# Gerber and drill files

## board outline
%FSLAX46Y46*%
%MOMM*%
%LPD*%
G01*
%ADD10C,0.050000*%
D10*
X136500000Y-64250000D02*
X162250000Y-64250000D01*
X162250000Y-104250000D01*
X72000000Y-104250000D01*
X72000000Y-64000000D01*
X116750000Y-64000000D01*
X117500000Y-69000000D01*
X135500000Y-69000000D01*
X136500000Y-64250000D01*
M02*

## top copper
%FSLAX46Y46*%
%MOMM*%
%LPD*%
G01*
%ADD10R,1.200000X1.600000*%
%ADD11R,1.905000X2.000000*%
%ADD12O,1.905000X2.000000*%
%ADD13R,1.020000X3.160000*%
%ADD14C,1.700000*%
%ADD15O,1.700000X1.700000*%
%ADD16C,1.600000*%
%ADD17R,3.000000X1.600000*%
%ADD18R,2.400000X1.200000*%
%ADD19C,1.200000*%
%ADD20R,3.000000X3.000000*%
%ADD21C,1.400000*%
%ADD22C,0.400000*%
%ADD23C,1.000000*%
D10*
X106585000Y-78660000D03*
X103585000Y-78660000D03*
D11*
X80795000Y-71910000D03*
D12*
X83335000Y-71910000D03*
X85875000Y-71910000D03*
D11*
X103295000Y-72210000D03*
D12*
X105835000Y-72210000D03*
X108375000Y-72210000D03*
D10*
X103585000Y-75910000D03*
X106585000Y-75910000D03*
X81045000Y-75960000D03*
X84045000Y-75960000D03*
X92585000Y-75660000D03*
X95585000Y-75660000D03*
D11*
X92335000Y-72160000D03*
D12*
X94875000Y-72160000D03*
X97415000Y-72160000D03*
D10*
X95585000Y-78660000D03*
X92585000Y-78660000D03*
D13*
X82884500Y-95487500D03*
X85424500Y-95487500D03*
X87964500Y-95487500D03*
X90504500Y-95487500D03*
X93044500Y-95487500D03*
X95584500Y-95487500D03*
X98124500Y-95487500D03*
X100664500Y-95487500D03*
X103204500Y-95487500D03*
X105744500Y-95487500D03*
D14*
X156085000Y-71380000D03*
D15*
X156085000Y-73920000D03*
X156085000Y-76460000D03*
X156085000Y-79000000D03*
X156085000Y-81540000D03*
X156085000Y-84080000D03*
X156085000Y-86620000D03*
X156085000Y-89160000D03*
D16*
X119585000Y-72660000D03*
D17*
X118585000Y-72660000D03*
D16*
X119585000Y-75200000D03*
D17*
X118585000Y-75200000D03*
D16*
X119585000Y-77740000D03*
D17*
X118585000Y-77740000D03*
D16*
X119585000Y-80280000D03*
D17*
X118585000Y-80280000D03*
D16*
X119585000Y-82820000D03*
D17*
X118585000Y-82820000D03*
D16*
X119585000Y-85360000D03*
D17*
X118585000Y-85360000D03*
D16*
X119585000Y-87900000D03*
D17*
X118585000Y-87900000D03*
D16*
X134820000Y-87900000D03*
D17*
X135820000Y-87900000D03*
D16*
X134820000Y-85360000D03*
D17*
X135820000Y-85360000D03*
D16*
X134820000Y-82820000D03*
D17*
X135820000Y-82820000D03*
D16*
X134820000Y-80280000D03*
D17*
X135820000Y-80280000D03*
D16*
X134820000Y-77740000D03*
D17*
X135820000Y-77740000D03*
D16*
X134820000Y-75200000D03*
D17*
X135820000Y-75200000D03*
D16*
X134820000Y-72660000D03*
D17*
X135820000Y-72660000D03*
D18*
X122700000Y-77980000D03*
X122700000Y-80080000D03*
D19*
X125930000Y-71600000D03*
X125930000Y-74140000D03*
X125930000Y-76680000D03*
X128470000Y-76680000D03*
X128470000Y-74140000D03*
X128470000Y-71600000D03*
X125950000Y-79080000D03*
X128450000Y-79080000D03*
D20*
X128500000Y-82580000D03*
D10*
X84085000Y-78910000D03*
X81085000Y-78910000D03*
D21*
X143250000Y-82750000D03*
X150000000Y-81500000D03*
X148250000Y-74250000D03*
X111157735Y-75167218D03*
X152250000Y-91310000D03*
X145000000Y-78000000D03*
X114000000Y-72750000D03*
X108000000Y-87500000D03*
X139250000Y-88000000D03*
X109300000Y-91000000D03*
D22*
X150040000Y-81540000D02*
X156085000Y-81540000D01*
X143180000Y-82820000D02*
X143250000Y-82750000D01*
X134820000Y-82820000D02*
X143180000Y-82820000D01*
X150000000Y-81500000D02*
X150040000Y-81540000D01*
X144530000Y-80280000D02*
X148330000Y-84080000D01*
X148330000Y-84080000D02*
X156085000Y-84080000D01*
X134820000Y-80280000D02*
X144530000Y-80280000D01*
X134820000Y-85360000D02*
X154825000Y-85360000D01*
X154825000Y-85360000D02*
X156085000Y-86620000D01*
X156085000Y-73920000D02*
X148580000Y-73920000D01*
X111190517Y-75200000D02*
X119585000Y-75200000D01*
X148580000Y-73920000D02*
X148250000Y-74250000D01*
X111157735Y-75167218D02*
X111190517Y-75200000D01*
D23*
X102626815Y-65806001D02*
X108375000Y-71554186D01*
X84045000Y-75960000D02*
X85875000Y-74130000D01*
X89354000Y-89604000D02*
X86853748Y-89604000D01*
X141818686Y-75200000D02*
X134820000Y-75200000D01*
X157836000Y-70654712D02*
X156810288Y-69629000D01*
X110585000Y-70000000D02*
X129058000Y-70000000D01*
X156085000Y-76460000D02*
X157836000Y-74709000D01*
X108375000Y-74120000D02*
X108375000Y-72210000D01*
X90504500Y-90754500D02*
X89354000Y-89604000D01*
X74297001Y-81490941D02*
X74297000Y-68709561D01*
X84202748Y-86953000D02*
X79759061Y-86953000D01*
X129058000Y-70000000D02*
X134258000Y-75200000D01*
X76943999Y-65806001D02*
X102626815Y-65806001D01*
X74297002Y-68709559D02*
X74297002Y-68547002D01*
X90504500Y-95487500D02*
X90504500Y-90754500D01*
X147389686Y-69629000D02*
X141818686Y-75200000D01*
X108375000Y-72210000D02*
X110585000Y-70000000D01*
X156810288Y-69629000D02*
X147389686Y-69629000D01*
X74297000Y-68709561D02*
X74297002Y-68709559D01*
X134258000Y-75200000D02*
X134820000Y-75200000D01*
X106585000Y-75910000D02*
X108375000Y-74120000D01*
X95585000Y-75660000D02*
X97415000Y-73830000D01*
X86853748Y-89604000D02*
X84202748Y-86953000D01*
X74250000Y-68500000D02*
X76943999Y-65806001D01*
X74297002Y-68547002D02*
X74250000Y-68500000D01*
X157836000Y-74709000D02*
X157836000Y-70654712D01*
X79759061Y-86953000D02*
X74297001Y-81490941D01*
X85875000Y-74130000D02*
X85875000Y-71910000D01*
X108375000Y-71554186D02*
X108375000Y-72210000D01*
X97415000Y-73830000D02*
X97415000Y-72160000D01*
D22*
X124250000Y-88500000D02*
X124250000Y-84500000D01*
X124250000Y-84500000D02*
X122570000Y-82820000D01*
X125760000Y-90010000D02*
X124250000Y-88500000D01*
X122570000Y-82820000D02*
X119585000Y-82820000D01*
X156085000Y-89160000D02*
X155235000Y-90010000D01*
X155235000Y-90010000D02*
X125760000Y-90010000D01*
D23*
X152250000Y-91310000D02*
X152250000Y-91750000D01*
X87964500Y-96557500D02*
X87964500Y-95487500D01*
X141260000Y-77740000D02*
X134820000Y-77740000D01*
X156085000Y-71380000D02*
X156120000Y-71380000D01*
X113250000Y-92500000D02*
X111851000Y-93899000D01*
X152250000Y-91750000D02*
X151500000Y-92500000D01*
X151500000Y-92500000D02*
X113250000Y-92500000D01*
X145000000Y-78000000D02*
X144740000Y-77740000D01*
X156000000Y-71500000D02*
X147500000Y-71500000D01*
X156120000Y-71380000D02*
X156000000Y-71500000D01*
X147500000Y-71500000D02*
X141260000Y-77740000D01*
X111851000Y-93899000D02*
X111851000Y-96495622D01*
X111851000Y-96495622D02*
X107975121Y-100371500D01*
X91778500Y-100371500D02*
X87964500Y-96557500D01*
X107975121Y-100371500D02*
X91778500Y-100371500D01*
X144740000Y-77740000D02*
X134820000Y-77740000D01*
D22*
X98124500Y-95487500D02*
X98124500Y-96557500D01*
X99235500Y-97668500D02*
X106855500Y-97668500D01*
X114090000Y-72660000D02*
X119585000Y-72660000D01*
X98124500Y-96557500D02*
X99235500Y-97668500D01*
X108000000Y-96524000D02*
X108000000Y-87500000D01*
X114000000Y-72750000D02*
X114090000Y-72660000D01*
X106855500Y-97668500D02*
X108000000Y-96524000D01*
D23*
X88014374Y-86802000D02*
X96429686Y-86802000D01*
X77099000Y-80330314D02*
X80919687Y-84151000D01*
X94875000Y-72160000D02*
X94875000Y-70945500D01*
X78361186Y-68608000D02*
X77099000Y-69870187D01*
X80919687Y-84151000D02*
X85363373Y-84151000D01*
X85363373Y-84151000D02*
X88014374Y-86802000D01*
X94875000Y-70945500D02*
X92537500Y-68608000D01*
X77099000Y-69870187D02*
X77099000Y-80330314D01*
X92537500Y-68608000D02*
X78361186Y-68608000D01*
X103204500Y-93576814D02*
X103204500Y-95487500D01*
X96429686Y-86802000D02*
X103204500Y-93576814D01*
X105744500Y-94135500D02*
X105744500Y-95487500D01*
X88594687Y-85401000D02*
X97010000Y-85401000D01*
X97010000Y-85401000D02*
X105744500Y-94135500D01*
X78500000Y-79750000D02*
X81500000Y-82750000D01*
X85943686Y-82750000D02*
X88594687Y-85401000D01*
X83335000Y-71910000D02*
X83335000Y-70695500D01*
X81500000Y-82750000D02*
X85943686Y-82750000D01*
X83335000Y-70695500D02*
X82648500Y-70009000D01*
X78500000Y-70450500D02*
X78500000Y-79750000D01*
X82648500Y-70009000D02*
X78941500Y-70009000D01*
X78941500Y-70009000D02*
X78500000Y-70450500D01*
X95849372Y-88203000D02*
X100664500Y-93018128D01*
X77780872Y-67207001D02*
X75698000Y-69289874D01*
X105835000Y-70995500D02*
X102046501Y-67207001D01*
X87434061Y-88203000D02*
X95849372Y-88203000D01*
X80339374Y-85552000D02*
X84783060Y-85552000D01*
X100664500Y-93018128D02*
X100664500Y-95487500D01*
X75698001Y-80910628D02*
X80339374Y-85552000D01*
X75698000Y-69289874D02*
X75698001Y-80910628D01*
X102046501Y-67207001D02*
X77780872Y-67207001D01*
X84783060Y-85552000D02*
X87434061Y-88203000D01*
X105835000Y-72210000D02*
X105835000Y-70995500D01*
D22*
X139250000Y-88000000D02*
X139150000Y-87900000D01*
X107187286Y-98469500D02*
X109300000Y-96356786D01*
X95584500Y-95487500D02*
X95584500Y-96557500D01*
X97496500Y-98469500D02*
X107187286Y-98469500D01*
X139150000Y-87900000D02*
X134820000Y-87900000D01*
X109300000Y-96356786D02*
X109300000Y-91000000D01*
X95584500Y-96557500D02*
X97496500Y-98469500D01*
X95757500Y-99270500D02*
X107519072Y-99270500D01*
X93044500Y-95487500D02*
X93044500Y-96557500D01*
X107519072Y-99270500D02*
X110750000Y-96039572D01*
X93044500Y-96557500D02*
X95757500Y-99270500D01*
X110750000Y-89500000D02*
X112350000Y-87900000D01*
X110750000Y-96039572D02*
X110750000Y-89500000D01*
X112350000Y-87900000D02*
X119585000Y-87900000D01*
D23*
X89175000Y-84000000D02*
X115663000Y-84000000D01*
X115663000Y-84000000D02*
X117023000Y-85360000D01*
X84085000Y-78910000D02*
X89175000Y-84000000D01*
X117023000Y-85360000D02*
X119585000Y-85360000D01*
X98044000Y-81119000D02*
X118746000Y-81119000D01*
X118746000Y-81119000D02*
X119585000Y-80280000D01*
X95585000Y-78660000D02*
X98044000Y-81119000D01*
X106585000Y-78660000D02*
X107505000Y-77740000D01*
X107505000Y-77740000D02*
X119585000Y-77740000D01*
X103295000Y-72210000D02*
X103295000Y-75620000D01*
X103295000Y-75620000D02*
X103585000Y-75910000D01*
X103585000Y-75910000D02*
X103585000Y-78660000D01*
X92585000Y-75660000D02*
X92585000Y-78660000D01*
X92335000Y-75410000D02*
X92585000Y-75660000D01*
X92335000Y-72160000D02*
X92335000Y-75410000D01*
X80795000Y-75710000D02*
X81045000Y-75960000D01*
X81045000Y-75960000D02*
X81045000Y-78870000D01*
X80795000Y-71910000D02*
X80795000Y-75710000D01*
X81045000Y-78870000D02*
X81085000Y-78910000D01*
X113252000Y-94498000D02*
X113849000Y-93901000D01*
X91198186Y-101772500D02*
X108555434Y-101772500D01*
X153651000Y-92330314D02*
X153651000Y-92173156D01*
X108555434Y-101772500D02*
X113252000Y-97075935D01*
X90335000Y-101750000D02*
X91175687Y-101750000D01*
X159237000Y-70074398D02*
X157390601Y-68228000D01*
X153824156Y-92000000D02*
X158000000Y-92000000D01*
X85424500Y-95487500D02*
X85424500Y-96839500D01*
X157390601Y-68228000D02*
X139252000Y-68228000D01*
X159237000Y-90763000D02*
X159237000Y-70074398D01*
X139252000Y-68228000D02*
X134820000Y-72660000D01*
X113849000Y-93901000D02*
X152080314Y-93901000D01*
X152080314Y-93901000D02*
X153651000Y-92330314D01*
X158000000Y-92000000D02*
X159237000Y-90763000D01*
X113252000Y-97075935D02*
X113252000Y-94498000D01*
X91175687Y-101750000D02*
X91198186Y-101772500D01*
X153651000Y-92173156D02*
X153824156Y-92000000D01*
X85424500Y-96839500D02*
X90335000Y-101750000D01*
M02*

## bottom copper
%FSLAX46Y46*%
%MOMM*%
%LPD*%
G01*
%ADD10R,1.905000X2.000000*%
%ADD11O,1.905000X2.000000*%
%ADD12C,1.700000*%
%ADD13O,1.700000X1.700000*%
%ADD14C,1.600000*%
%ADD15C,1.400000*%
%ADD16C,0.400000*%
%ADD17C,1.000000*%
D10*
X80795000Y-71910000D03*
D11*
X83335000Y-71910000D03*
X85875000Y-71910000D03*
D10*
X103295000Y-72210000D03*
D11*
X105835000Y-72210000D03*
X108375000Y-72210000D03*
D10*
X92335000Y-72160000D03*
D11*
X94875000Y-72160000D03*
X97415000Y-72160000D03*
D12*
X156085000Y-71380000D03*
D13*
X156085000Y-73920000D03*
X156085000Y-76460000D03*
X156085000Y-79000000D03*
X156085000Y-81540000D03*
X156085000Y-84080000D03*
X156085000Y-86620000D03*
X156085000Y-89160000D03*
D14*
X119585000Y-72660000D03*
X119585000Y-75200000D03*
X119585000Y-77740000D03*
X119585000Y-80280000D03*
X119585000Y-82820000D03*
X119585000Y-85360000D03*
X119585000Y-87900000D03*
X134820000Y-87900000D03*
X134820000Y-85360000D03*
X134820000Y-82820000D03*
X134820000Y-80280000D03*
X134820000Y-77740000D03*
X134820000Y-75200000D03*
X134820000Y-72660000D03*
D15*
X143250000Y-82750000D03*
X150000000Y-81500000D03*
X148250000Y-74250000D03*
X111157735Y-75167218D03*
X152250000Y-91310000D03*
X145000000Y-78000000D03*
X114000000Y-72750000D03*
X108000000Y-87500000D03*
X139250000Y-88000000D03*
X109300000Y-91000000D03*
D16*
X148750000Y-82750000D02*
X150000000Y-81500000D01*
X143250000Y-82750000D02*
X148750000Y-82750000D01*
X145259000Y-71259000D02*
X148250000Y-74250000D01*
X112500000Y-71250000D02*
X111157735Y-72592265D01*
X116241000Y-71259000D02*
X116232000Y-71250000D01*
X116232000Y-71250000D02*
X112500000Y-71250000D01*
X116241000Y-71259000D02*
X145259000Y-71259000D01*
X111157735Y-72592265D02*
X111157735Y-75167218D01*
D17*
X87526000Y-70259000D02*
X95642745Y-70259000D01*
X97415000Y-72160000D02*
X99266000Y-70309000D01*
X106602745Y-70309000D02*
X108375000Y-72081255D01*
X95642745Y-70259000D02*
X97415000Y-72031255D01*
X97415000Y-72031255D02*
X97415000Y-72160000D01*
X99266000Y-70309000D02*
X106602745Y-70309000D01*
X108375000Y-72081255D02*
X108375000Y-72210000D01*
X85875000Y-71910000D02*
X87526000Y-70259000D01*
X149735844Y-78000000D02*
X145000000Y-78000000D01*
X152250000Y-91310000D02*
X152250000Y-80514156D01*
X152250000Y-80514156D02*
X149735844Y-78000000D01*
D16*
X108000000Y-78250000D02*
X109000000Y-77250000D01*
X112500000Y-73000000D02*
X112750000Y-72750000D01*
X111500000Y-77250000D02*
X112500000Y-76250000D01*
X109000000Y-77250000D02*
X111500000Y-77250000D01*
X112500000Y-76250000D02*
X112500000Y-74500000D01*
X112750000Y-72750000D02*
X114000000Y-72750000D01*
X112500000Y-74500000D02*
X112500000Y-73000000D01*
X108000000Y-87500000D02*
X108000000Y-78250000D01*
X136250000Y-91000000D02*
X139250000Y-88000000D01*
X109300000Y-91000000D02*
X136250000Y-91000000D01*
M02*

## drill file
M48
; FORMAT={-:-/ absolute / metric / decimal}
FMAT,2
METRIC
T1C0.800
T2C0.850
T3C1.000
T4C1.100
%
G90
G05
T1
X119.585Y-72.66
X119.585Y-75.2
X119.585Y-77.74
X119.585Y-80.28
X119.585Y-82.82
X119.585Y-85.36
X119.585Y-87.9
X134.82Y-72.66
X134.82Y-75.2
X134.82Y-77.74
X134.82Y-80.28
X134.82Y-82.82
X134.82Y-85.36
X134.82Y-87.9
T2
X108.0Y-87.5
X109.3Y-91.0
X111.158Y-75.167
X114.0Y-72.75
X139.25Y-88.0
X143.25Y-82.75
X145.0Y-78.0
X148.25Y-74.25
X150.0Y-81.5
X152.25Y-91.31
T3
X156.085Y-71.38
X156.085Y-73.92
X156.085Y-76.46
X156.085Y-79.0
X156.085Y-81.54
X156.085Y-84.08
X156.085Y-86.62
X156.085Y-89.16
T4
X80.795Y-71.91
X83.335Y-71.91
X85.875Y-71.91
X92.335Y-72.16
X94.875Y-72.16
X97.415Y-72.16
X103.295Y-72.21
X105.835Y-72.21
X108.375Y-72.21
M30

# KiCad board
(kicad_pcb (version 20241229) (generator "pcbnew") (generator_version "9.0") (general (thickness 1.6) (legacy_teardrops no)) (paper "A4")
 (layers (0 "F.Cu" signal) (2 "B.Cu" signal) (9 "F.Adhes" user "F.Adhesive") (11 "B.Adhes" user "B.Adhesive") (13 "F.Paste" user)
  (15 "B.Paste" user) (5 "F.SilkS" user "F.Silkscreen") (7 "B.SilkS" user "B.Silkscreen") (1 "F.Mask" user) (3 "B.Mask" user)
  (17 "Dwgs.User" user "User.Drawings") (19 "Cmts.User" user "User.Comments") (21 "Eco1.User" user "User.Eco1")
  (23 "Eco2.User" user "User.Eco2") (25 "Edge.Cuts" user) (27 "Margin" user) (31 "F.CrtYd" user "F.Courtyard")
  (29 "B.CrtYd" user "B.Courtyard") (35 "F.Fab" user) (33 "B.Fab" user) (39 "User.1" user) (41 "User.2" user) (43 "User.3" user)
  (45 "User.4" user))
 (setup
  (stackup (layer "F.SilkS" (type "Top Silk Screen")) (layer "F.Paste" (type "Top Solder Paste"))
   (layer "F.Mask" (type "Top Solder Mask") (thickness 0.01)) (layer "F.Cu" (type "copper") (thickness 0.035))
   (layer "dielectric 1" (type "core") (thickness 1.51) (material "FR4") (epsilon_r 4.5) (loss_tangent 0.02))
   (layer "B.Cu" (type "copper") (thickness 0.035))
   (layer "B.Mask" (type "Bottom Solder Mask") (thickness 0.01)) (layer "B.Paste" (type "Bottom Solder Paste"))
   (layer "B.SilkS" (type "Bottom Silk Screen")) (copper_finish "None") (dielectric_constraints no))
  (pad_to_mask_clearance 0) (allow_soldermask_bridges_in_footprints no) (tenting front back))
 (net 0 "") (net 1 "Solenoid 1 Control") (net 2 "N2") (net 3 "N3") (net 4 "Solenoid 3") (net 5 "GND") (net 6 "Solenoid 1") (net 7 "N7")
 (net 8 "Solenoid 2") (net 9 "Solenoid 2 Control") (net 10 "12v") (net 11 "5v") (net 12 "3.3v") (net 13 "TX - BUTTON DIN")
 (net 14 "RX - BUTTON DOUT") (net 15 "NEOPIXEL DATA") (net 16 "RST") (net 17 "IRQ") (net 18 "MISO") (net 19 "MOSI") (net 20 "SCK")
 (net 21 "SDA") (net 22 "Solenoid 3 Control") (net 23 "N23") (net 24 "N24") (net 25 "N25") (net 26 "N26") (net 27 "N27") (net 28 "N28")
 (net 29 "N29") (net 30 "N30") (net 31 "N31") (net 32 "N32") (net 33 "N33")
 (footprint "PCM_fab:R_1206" (layer "F.Cu") (at 105.085 78.66 180)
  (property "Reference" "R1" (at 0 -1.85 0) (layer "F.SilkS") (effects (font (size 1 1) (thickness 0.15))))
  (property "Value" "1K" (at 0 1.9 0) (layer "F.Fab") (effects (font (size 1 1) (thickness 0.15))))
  (pad "1" smd rect (at -1.5 0 180) (size 1.2 1.6) (layers "F.Cu" "F.Mask" "F.Paste") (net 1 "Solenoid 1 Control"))
  (pad "2" smd rect (at 1.5 0 180) (size 1.2 1.6) (layers "F.Cu" "F.Mask" "F.Paste") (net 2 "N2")))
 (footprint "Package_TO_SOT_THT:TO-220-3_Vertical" (layer "F.Cu") (at 80.795 71.91)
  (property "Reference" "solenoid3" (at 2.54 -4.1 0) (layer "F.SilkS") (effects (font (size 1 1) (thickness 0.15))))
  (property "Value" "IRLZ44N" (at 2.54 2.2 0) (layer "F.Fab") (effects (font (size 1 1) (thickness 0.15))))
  (pad "1" thru_hole rect (at 0 0) (size 1.905 2) (drill 1.1) (layers "*.Cu" "*.Mask") (remove_unused_layers no) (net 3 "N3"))
  (pad "2" thru_hole oval (at 2.54 0) (size 1.905 2) (drill 1.1) (layers "*.Cu" "*.Mask") (remove_unused_layers no) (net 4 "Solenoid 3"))
  (pad "3" thru_hole oval (at 5.08 0) (size 1.905 2) (drill 1.1) (layers "*.Cu" "*.Mask") (remove_unused_layers no) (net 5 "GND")))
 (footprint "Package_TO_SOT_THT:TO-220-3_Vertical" (layer "F.Cu") (at 103.295 72.21)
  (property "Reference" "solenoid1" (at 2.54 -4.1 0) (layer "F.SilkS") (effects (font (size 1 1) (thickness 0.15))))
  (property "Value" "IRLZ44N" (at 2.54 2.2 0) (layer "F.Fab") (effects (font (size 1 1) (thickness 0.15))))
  (pad "1" thru_hole rect (at 0 0) (size 1.905 2) (drill 1.1) (layers "*.Cu" "*.Mask") (remove_unused_layers no) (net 2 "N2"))
  (pad "2" thru_hole oval (at 2.54 0) (size 1.905 2) (drill 1.1) (layers "*.Cu" "*.Mask") (remove_unused_layers no) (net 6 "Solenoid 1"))
  (pad "3" thru_hole oval (at 5.08 0) (size 1.905 2) (drill 1.1) (layers "*.Cu" "*.Mask") (remove_unused_layers no) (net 5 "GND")))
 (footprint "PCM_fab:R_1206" (layer "F.Cu") (at 105.085 75.91)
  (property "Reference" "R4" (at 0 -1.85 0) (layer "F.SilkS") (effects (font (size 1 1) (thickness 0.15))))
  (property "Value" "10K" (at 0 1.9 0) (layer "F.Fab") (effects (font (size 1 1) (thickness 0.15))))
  (pad "1" smd rect (at -1.5 0) (size 1.2 1.6) (layers "F.Cu" "F.Mask" "F.Paste") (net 2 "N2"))
  (pad "2" smd rect (at 1.5 0) (size 1.2 1.6) (layers "F.Cu" "F.Mask" "F.Paste") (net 5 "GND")))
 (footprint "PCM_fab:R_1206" (layer "F.Cu") (at 82.545 75.96)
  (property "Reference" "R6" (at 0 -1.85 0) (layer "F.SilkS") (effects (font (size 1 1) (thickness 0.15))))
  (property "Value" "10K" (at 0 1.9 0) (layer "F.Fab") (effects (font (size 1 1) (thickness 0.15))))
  (pad "1" smd rect (at -1.5 0) (size 1.2 1.6) (layers "F.Cu" "F.Mask" "F.Paste") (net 3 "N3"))
  (pad "2" smd rect (at 1.5 0) (size 1.2 1.6) (layers "F.Cu" "F.Mask" "F.Paste") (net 5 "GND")))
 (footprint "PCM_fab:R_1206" (layer "F.Cu") (at 94.085 75.66)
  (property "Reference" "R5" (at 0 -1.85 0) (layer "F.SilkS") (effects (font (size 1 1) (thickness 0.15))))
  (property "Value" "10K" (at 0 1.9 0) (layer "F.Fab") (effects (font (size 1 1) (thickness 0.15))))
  (pad "1" smd rect (at -1.5 0) (size 1.2 1.6) (layers "F.Cu" "F.Mask" "F.Paste") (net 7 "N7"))
  (pad "2" smd rect (at 1.5 0) (size 1.2 1.6) (layers "F.Cu" "F.Mask" "F.Paste") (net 5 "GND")))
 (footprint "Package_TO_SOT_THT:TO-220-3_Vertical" (layer "F.Cu") (at 92.335 72.16)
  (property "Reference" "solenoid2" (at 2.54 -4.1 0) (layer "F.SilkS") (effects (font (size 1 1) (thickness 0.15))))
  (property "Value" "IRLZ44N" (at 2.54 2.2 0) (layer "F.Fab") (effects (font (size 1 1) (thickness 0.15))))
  (pad "1" thru_hole rect (at 0 0) (size 1.905 2) (drill 1.1) (layers "*.Cu" "*.Mask") (remove_unused_layers no) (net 7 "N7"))
  (pad "2" thru_hole oval (at 2.54 0) (size 1.905 2) (drill 1.1) (layers "*.Cu" "*.Mask") (remove_unused_layers no) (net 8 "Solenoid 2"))
  (pad "3" thru_hole oval (at 5.08 0) (size 1.905 2) (drill 1.1) (layers "*.Cu" "*.Mask") (remove_unused_layers no) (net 5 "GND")))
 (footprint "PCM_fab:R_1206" (layer "F.Cu") (at 94.085 78.66 180)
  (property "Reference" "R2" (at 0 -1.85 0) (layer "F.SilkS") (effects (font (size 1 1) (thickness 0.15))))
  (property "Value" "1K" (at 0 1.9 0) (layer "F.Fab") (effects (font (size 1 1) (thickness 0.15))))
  (pad "1" smd rect (at -1.5 0 180) (size 1.2 1.6) (layers "F.Cu" "F.Mask" "F.Paste") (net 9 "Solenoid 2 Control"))
  (pad "2" smd rect (at 1.5 0 180) (size 1.2 1.6) (layers "F.Cu" "F.Mask" "F.Paste") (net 7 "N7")))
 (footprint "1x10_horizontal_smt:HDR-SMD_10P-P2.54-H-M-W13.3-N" (layer "F.Cu") (at 94.3145 95.4875)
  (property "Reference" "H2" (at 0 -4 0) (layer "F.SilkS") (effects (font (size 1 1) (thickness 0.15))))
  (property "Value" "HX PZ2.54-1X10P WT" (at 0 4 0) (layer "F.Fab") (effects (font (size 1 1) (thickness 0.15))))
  (pad "1" smd rect (at -11.43 0) (size 1.02 3.16) (layers "F.Cu" "F.Mask" "F.Paste") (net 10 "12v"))
  (pad "2" smd rect (at -8.89 0) (size 1.02 3.16) (layers "F.Cu" "F.Mask" "F.Paste") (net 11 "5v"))
  (pad "3" smd rect (at -6.35 0) (size 1.02 3.16) (layers "F.Cu" "F.Mask" "F.Paste") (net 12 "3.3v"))
  (pad "4" smd rect (at -3.81 0) (size 1.02 3.16) (layers "F.Cu" "F.Mask" "F.Paste") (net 5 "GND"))
  (pad "5" smd rect (at -1.27 0) (size 1.02 3.16) (layers "F.Cu" "F.Mask" "F.Paste") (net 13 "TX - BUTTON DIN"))
  (pad "6" smd rect (at 1.27 0) (size 1.02 3.16) (layers "F.Cu" "F.Mask" "F.Paste") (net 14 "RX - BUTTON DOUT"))
  (pad "7" smd rect (at 3.81 0) (size 1.02 3.16) (layers "F.Cu" "F.Mask" "F.Paste") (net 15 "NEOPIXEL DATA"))
  (pad "8" smd rect (at 6.35 0) (size 1.02 3.16) (layers "F.Cu" "F.Mask" "F.Paste") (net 6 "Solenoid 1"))
  (pad "9" smd rect (at 8.89 0) (size 1.02 3.16) (layers "F.Cu" "F.Mask" "F.Paste") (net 8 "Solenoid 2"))
  (pad "10" smd rect (at 11.43 0) (size 1.02 3.16) (layers "F.Cu" "F.Mask" "F.Paste") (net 4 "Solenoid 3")))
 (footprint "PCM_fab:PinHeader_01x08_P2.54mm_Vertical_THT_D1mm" (layer "F.Cu") (at 156.085 71.38)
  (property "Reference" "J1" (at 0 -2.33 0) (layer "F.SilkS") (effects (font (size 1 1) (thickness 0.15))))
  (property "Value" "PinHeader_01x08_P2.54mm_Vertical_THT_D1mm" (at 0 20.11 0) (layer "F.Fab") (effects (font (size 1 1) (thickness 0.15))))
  (pad "1" thru_hole circle (at 0 0) (size 1.7 1.7) (drill 1) (layers "*.Cu" "*.Mask") (remove_unused_layers no) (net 12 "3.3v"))
  (pad "2" thru_hole oval (at 0 2.54) (size 1.7 1.7) (drill 1) (layers "*.Cu" "*.Mask") (remove_unused_layers no) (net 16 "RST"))
  (pad "3" thru_hole oval (at 0 5.08) (size 1.7 1.7) (drill 1) (layers "*.Cu" "*.Mask") (remove_unused_layers no) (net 5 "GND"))
  (pad "4" thru_hole oval (at 0 7.62) (size 1.7 1.7) (drill 1) (layers "*.Cu" "*.Mask") (remove_unused_layers no) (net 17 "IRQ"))
  (pad "5" thru_hole oval (at 0 10.16) (size 1.7 1.7) (drill 1) (layers "*.Cu" "*.Mask") (remove_unused_layers no) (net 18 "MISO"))
  (pad "6" thru_hole oval (at 0 12.7) (size 1.7 1.7) (drill 1) (layers "*.Cu" "*.Mask") (remove_unused_layers no) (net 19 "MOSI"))
  (pad "7" thru_hole oval (at 0 15.24) (size 1.7 1.7) (drill 1) (layers "*.Cu" "*.Mask") (remove_unused_layers no) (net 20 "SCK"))
  (pad "8" thru_hole oval (at 0 17.78) (size 1.7 1.7) (drill 1) (layers "*.Cu" "*.Mask") (remove_unused_layers no) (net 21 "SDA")))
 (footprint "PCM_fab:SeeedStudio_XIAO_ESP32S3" (layer "F.Cu") (at 127.2 80.28)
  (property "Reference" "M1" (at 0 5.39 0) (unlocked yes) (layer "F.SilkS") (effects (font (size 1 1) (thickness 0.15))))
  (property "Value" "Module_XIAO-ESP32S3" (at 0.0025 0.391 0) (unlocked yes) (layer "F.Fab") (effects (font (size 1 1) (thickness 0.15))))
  (pad "1" thru_hole circle (at -7.615 -7.62) (size 1.6 1.6) (drill 0.8) (layers "*.Cu" "*.Mask") (remove_unused_layers no)
   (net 15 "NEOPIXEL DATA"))
  (pad "1" smd rect (at -7.615 -7.62) (size 3 1.6) (drill (offset -1 0)) (layers "F.Cu" "F.Mask" "F.Paste") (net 15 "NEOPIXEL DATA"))
  (pad "2" thru_hole circle (at -7.615 -5.08) (size 1.6 1.6) (drill 0.8) (layers "*.Cu" "*.Mask") (remove_unused_layers no) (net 16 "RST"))
  (pad "2" smd rect (at -7.615 -5.08) (size 3 1.6) (drill (offset -1 0)) (layers "F.Cu" "F.Mask" "F.Paste") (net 16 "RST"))
  (pad "3" thru_hole circle (at -7.615 -2.54) (size 1.6 1.6) (drill 0.8) (layers "*.Cu" "*.Mask") (remove_unused_layers no)
   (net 1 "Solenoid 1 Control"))
  (pad "3" smd rect (at -7.615 -2.54) (size 3 1.6) (drill (offset -1 0)) (layers "F.Cu" "F.Mask" "F.Paste") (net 1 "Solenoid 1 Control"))
  (pad "4" thru_hole circle (at -7.615 0) (size 1.6 1.6) (drill 0.8) (layers "*.Cu" "*.Mask") (remove_unused_layers no)
   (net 9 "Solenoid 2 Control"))
  (pad "4" smd rect (at -7.615 0) (size 3 1.6) (drill (offset -1 0)) (layers "F.Cu" "F.Mask" "F.Paste") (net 9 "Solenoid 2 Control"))
  (pad "5" thru_hole circle (at -7.615 2.54) (size 1.6 1.6) (drill 0.8) (layers "*.Cu" "*.Mask") (remove_unused_layers no) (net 21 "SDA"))
  (pad "5" smd rect (at -7.615 2.54) (size 3 1.6) (drill (offset -1 0)) (layers "F.Cu" "F.Mask" "F.Paste") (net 21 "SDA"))
  (pad "6" thru_hole circle (at -7.615 5.08) (size 1.6 1.6) (drill 0.8) (layers "*.Cu" "*.Mask") (remove_unused_layers no)
   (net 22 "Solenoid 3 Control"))
  (pad "6" smd rect (at -7.615 5.08) (size 3 1.6) (drill (offset -1 0)) (layers "F.Cu" "F.Mask" "F.Paste") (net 22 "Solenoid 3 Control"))
  (pad "7" thru_hole circle (at -7.615 7.62) (size 1.6 1.6) (drill 0.8) (layers "*.Cu" "*.Mask") (remove_unused_layers no)
   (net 13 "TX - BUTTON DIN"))
  (pad "7" smd rect (at -7.615 7.62) (size 3 1.6) (drill (offset -1 0)) (layers "F.Cu" "F.Mask" "F.Paste") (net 13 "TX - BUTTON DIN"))
  (pad "8" thru_hole circle (at 7.62 7.62) (size 1.6 1.6) (drill 0.8) (layers "*.Cu" "*.Mask") (remove_unused_layers no)
   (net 14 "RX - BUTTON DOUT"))
  (pad "8" smd rect (at 7.62 7.62) (size 3 1.6) (drill (offset 1 0)) (layers "F.Cu" "F.Mask" "F.Paste") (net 14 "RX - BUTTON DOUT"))
  (pad "9" thru_hole circle (at 7.62 5.08) (size 1.6 1.6) (drill 0.8) (layers "*.Cu" "*.Mask") (remove_unused_layers no) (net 20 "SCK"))
  (pad "9" smd rect (at 7.62 5.08) (size 3 1.6) (drill (offset 1 0)) (layers "F.Cu" "F.Mask" "F.Paste") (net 20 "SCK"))
  (pad "10" thru_hole circle (at 7.62 2.54) (size 1.6 1.6) (drill 0.8) (layers "*.Cu" "*.Mask") (remove_unused_layers no) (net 18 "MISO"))
  (pad "10" smd rect (at 7.62 2.54) (size 3 1.6) (drill (offset 1 0)) (layers "F.Cu" "F.Mask" "F.Paste") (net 18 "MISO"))
  (pad "11" thru_hole circle (at 7.62 0) (size 1.6 1.6) (drill 0.8) (layers "*.Cu" "*.Mask") (remove_unused_layers no) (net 19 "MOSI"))
  (pad "11" smd rect (at 7.62 0) (size 3 1.6) (drill (offset 1 0)) (layers "F.Cu" "F.Mask" "F.Paste") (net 19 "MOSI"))
  (pad "12" thru_hole circle (at 7.62 -2.54) (size 1.6 1.6) (drill 0.8) (layers "*.Cu" "*.Mask") (remove_unused_layers no) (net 12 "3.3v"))
  (pad "12" smd rect (at 7.62 -2.54) (size 3 1.6) (drill (offset 1 0)) (layers "F.Cu" "F.Mask" "F.Paste") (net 12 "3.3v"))
  (pad "13" thru_hole circle (at 7.62 -5.08) (size 1.6 1.6) (drill 0.8) (layers "*.Cu" "*.Mask") (remove_unused_layers no) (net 5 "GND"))
  (pad "13" smd rect (at 7.62 -5.08) (size 3 1.6) (drill (offset 1 0)) (layers "F.Cu" "F.Mask" "F.Paste") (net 5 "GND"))
  (pad "14" thru_hole circle (at 7.62 -7.62) (size 1.6 1.6) (drill 0.8) (layers "*.Cu" "*.Mask") (remove_unused_layers no) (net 11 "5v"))
  (pad "14" smd rect (at 7.62 -7.62) (size 3 1.6) (drill (offset 1 0)) (layers "F.Cu" "F.Mask" "F.Paste") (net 11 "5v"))
  (pad "15" smd rect (at -4.5 -2.3) (size 2.4 1.2) (layers "F.Cu" "F.Mask" "F.Paste") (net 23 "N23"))
  (pad "16" smd rect (at -4.5 -0.2) (size 2.4 1.2) (layers "F.Cu" "F.Mask" "F.Paste") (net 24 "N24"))
  (pad "17" smd circle (at -1.27 -8.68) (size 1.2 1.2) (layers "F.Cu" "F.Mask" "F.Paste") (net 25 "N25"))
  (pad "18" smd circle (at -1.27 -6.14) (size 1.2 1.2) (layers "F.Cu" "F.Mask" "F.Paste") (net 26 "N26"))
  (pad "19" smd circle (at -1.27 -3.6) (size 1.2 1.2) (layers "F.Cu" "F.Mask" "F.Paste") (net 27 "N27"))
  (pad "20" smd circle (at 1.27 -3.6) (size 1.2 1.2) (layers "F.Cu" "F.Mask" "F.Paste") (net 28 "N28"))
  (pad "21" smd circle (at 1.27 -6.14) (size 1.2 1.2) (layers "F.Cu" "F.Mask" "F.Paste") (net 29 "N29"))
  (pad "22" smd circle (at 1.27 -8.68) (size 1.2 1.2) (layers "F.Cu" "F.Mask" "F.Paste") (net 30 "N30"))
  (pad "23" smd circle (at -1.25 -1.2) (size 1.2 1.2) (layers "F.Cu" "F.Mask" "F.Paste") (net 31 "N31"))
  (pad "24" smd circle (at 1.25 -1.2) (size 1.2 1.2) (layers "F.Cu" "F.Mask" "F.Paste") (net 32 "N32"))
  (pad "25" smd rect (at 1.3 2.3) (size 3 3) (layers "F.Cu" "F.Mask" "F.Paste") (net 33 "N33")))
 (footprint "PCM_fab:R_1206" (layer "F.Cu") (at 82.585 78.91 180)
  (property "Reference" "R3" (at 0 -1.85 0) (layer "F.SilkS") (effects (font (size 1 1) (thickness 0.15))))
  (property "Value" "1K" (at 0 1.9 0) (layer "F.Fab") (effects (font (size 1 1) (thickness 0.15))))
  (pad "1" smd rect (at -1.5 0 180) (size 1.2 1.6) (layers "F.Cu" "F.Mask" "F.Paste") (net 22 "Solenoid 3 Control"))
  (pad "2" smd rect (at 1.5 0 180) (size 1.2 1.6) (layers "F.Cu" "F.Mask" "F.Paste") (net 3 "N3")))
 (gr_poly
  (pts (xy 136.5 64.25) (xy 162.25 64.25) (xy 162.25 104.25) (xy 72 104.25) (xy 72 64) (xy 116.75 64) (xy 117.5 69) (xy 135.5 69))
  (stroke (width 0.05) (type solid)) (fill no) (layer "Edge.Cuts"))
 (segment (start 150.04 81.54) (end 156.085 81.54) (width 0.4) (layer "F.Cu") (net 18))
 (segment (start 143.18 82.82) (end 143.25 82.75) (width 0.4) (layer "F.Cu") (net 18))
 (segment (start 134.82 82.82) (end 143.18 82.82) (width 0.4) (layer "F.Cu") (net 18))
 (segment (start 150 81.5) (end 150.04 81.54) (width 0.4) (layer "F.Cu") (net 18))
 (via (at 143.25 82.75) (size 1.4) (drill 0.85) (layers "F.Cu" "B.Cu") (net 18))
 (via (at 150 81.5) (size 1.4) (drill 0.85) (layers "F.Cu" "B.Cu") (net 18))
 (segment (start 148.75 82.75) (end 150 81.5) (width 0.4) (layer "B.Cu") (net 18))
 (segment (start 143.25 82.75) (end 148.75 82.75) (width 0.4) (layer "B.Cu") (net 18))
 (segment (start 144.53 80.28) (end 148.33 84.08) (width 0.4) (layer "F.Cu") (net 19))
 (segment (start 148.33 84.08) (end 156.085 84.08) (width 0.4) (layer "F.Cu") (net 19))
 (segment (start 134.82 80.28) (end 144.53 80.28) (width 0.4) (layer "F.Cu") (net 19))
 (segment (start 134.82 85.36) (end 154.825 85.36) (width 0.4) (layer "F.Cu") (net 20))
 (segment (start 154.825 85.36) (end 156.085 86.62) (width 0.4) (layer "F.Cu") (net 20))
 (segment (start 156.085 73.92) (end 148.58 73.92) (width 0.4) (layer "F.Cu") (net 16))
 (segment (start 111.190517 75.2) (end 119.585 75.2) (width 0.4) (layer "F.Cu") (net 16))
 (segment (start 148.58 73.92) (end 148.25 74.25) (width 0.4) (layer "F.Cu") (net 16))
 (segment (start 111.157735 75.167218) (end 111.190517 75.2) (width 0.4) (layer "F.Cu") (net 16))
 (via (at 148.25 74.25) (size 1.4) (drill 0.85) (layers "F.Cu" "B.Cu") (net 16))
 (via (at 111.157735 75.167218) (size 1.4) (drill 0.85) (layers "F.Cu" "B.Cu") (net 16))
 (segment (start 145.259 71.259) (end 148.25 74.25) (width 0.4) (layer "B.Cu") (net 16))
 (segment (start 112.5 71.25) (end 111.157735 72.592265) (width 0.4) (layer "B.Cu") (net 16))
 (segment (start 116.241 71.259) (end 116.232 71.25) (width 0.4) (layer "B.Cu") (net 16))
 (segment (start 116.232 71.25) (end 112.5 71.25) (width 0.4) (layer "B.Cu") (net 16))
 (segment (start 116.241 71.259) (end 145.259 71.259) (width 0.4) (layer "B.Cu") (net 16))
 (segment (start 111.157735 72.592265) (end 111.157735 75.167218) (width 0.4) (layer "B.Cu") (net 16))
 (segment (start 102.626815 65.806001) (end 108.375 71.554186) (width 1) (layer "F.Cu") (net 5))
 (segment (start 84.045 75.96) (end 85.875 74.13) (width 1) (layer "F.Cu") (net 5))
 (segment (start 89.354 89.604) (end 86.853748 89.604) (width 1) (layer "F.Cu") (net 5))
 (segment (start 141.818686 75.2) (end 134.82 75.2) (width 1) (layer "F.Cu") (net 5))
 (segment (start 157.836 70.654712) (end 156.810288 69.629) (width 1) (layer "F.Cu") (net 5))
 (segment (start 110.585 70) (end 129.058 70) (width 1) (layer "F.Cu") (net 5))
 (segment (start 156.085 76.46) (end 157.836 74.709) (width 1) (layer "F.Cu") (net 5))
 (segment (start 108.375 74.12) (end 108.375 72.21) (width 1) (layer "F.Cu") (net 5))
 (segment (start 90.5045 90.7545) (end 89.354 89.604) (width 1) (layer "F.Cu") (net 5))
 (segment (start 74.297001 81.490941) (end 74.297 68.709561) (width 1) (layer "F.Cu") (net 5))
 (segment (start 84.202748 86.953) (end 79.759061 86.953) (width 1) (layer "F.Cu") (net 5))
 (segment (start 129.058 70) (end 134.258 75.2) (width 1) (layer "F.Cu") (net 5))
 (segment (start 76.943999 65.806001) (end 102.626815 65.806001) (width 1) (layer "F.Cu") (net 5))
 (segment (start 74.297002 68.709559) (end 74.297002 68.547002) (width 1) (layer "F.Cu") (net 5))
 (segment (start 90.5045 95.4875) (end 90.5045 90.7545) (width 1) (layer "F.Cu") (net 5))
 (segment (start 147.389686 69.629) (end 141.818686 75.2) (width 1) (layer "F.Cu") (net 5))
 (segment (start 108.375 72.21) (end 110.585 70) (width 1) (layer "F.Cu") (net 5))
 (segment (start 156.810288 69.629) (end 147.389686 69.629) (width 1) (layer "F.Cu") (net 5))
 (segment (start 74.297 68.709561) (end 74.297002 68.709559) (width 1) (layer "F.Cu") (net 5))
 (segment (start 134.258 75.2) (end 134.82 75.2) (width 1) (layer "F.Cu") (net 5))
 (segment (start 106.585 75.91) (end 108.375 74.12) (width 1) (layer "F.Cu") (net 5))
 (segment (start 95.585 75.66) (end 97.415 73.83) (width 1) (layer "F.Cu") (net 5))
 (segment (start 86.853748 89.604) (end 84.202748 86.953) (width 1) (layer "F.Cu") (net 5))
 (segment (start 74.25 68.5) (end 76.943999 65.806001) (width 1) (layer "F.Cu") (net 5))
 (segment (start 74.297002 68.547002) (end 74.25 68.5) (width 1) (layer "F.Cu") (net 5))
 (segment (start 157.836 74.709) (end 157.836 70.654712) (width 1) (layer "F.Cu") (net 5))
 (segment (start 79.759061 86.953) (end 74.297001 81.490941) (width 1) (layer "F.Cu") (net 5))
 (segment (start 85.875 74.13) (end 85.875 71.91) (width 1) (layer "F.Cu") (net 5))
 (segment (start 108.375 71.554186) (end 108.375 72.21) (width 1) (layer "F.Cu") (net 5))
 (segment (start 97.415 73.83) (end 97.415 72.16) (width 1) (layer "F.Cu") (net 5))
 (segment (start 87.526 70.259) (end 95.642745 70.259) (width 1) (layer "B.Cu") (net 5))
 (segment (start 97.415 72.16) (end 99.266 70.309) (width 1) (layer "B.Cu") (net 5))
 (segment (start 106.602745 70.309) (end 108.375 72.081255) (width 1) (layer "B.Cu") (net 5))
 (segment (start 95.642745 70.259) (end 97.415 72.031255) (width 1) (layer "B.Cu") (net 5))
 (segment (start 97.415 72.031255) (end 97.415 72.16) (width 1) (layer "B.Cu") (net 5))
 (segment (start 99.266 70.309) (end 106.602745 70.309) (width 1) (layer "B.Cu") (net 5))
 (segment (start 108.375 72.081255) (end 108.375 72.21) (width 1) (layer "B.Cu") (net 5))
 (segment (start 85.875 71.91) (end 87.526 70.259) (width 1) (layer "B.Cu") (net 5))
 (segment (start 124.25 88.5) (end 124.25 84.5) (width 0.4) (layer "F.Cu") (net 21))
 (segment (start 124.25 84.5) (end 122.57 82.82) (width 0.4) (layer "F.Cu") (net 21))
 (segment (start 125.76 90.01) (end 124.25 88.5) (width 0.4) (layer "F.Cu") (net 21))
 (segment (start 122.57 82.82) (end 119.585 82.82) (width 0.4) (layer "F.Cu") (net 21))
 (segment (start 156.085 89.16) (end 155.235 90.01) (width 0.4) (layer "F.Cu") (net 21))
 (segment (start 155.235 90.01) (end 125.76 90.01) (width 0.4) (layer "F.Cu") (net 21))
 (segment (start 152.25 91.31) (end 152.25 91.75) (width 1) (layer "F.Cu") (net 12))
 (segment (start 87.9645 96.5575) (end 87.9645 95.4875) (width 1) (layer "F.Cu") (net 12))
 (segment (start 141.26 77.74) (end 134.82 77.74) (width 1) (layer "F.Cu") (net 12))
 (segment (start 156.085 71.38) (end 156.12 71.38) (width 1) (layer "F.Cu") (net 12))
 (segment (start 113.25 92.5) (end 111.851 93.899) (width 1) (layer "F.Cu") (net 12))
 (segment (start 152.25 91.75) (end 151.5 92.5) (width 1) (layer "F.Cu") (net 12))
 (segment (start 151.5 92.5) (end 113.25 92.5) (width 1) (layer "F.Cu") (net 12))
 (segment (start 145 78) (end 144.74 77.74) (width 1) (layer "F.Cu") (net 12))
 (segment (start 156 71.5) (end 147.5 71.5) (width 1) (layer "F.Cu") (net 12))
 (segment (start 156.12 71.38) (end 156 71.5) (width 1) (layer "F.Cu") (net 12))
 (segment (start 147.5 71.5) (end 141.26 77.74) (width 1) (layer "F.Cu") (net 12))
 (segment (start 111.851 93.899) (end 111.851 96.495622) (width 1) (layer "F.Cu") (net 12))
 (segment (start 111.851 96.495622) (end 107.975121 100.3715) (width 1) (layer "F.Cu") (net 12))
 (segment (start 91.7785 100.3715) (end 87.9645 96.5575) (width 1) (layer "F.Cu") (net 12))
 (segment (start 107.975121 100.3715) (end 91.7785 100.3715) (width 1) (layer "F.Cu") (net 12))
 (segment (start 144.74 77.74) (end 134.82 77.74) (width 1) (layer "F.Cu") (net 12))
 (via (at 152.25 91.31) (size 1.4) (drill 0.85) (layers "F.Cu" "B.Cu") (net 12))
 (via (at 145 78) (size 1.4) (drill 0.85) (layers "F.Cu" "B.Cu") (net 12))
 (segment (start 149.735844 78) (end 145 78) (width 1) (layer "B.Cu") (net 12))
 (segment (start 152.25 91.31) (end 152.25 80.514156) (width 1) (layer "B.Cu") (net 12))
 (segment (start 152.25 80.514156) (end 149.735844 78) (width 1) (layer "B.Cu") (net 12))
 (segment (start 98.1245 95.4875) (end 98.1245 96.5575) (width 0.4) (layer "F.Cu") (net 15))
 (segment (start 99.2355 97.6685) (end 106.8555 97.6685) (width 0.4) (layer "F.Cu") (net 15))
 (segment (start 114.09 72.66) (end 119.585 72.66) (width 0.4) (layer "F.Cu") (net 15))
 (segment (start 98.1245 96.5575) (end 99.2355 97.6685) (width 0.4) (layer "F.Cu") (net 15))
 (segment (start 108 96.524) (end 108 87.5) (width 0.4) (layer "F.Cu") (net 15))
 (segment (start 114 72.75) (end 114.09 72.66) (width 0.4) (layer "F.Cu") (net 15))
 (segment (start 106.8555 97.6685) (end 108 96.524) (width 0.4) (layer "F.Cu") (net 15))
 (via (at 114 72.75) (size 1.4) (drill 0.85) (layers "F.Cu" "B.Cu") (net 15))
 (via (at 108 87.5) (size 1.4) (drill 0.85) (layers "F.Cu" "B.Cu") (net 15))
 (segment (start 108 78.25) (end 109 77.25) (width 0.4) (layer "B.Cu") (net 15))
 (segment (start 112.5 73) (end 112.75 72.75) (width 0.4) (layer "B.Cu") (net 15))
 (segment (start 111.5 77.25) (end 112.5 76.25) (width 0.4) (layer "B.Cu") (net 15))
 (segment (start 109 77.25) (end 111.5 77.25) (width 0.4) (layer "B.Cu") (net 15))
 (segment (start 112.5 76.25) (end 112.5 74.5) (width 0.4) (layer "B.Cu") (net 15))
 (segment (start 112.75 72.75) (end 114 72.75) (width 0.4) (layer "B.Cu") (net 15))
 (segment (start 112.5 74.5) (end 112.5 73) (width 0.4) (layer "B.Cu") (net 15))
 (segment (start 108 87.5) (end 108 78.25) (width 0.4) (layer "B.Cu") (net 15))
 (segment (start 88.014374 86.802) (end 96.429686 86.802) (width 1) (layer "F.Cu") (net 8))
 (segment (start 77.099 80.330314) (end 80.919687 84.151) (width 1) (layer "F.Cu") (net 8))
 (segment (start 94.875 72.16) (end 94.875 70.9455) (width 1) (layer "F.Cu") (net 8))
 (segment (start 78.361186 68.608) (end 77.099 69.870187) (width 1) (layer "F.Cu") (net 8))
 (segment (start 80.919687 84.151) (end 85.363373 84.151) (width 1) (layer "F.Cu") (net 8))
 (segment (start 85.363373 84.151) (end 88.014374 86.802) (width 1) (layer "F.Cu") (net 8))
 (segment (start 94.875 70.9455) (end 92.5375 68.608) (width 1) (layer "F.Cu") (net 8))
 (segment (start 77.099 69.870187) (end 77.099 80.330314) (width 1) (layer "F.Cu") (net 8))
 (segment (start 92.5375 68.608) (end 78.361186 68.608) (width 1) (layer "F.Cu") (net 8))
 (segment (start 103.2045 93.576814) (end 103.2045 95.4875) (width 1) (layer "F.Cu") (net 8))
 (segment (start 96.429686 86.802) (end 103.2045 93.576814) (width 1) (layer "F.Cu") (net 8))
 (segment (start 105.7445 94.1355) (end 105.7445 95.4875) (width 1) (layer "F.Cu") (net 4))
 (segment (start 88.594687 85.401) (end 97.01 85.401) (width 1) (layer "F.Cu") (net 4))
 (segment (start 97.01 85.401) (end 105.7445 94.1355) (width 1) (layer "F.Cu") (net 4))
 (segment (start 78.5 79.75) (end 81.5 82.75) (width 1) (layer "F.Cu") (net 4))
 (segment (start 85.943686 82.75) (end 88.594687 85.401) (width 1) (layer "F.Cu") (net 4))
 (segment (start 83.335 71.91) (end 83.335 70.6955) (width 1) (layer "F.Cu") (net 4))
 (segment (start 81.5 82.75) (end 85.943686 82.75) (width 1) (layer "F.Cu") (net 4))
 (segment (start 83.335 70.6955) (end 82.6485 70.009) (width 1) (layer "F.Cu") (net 4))
 (segment (start 78.5 70.4505) (end 78.5 79.75) (width 1) (layer "F.Cu") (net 4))
 (segment (start 82.6485 70.009) (end 78.9415 70.009) (width 1) (layer "F.Cu") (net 4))
 (segment (start 78.9415 70.009) (end 78.5 70.4505) (width 1) (layer "F.Cu") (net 4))
 (segment (start 95.849372 88.203) (end 100.6645 93.018128) (width 1) (layer "F.Cu") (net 6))
 (segment (start 77.780872 67.207001) (end 75.698 69.289874) (width 1) (layer "F.Cu") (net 6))
 (segment (start 105.835 70.9955) (end 102.046501 67.207001) (width 1) (layer "F.Cu") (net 6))
 (segment (start 87.434061 88.203) (end 95.849372 88.203) (width 1) (layer "F.Cu") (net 6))
 (segment (start 80.339374 85.552) (end 84.78306 85.552) (width 1) (layer "F.Cu") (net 6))
 (segment (start 100.6645 93.018128) (end 100.6645 95.4875) (width 1) (layer "F.Cu") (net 6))
 (segment (start 75.698001 80.910628) (end 80.339374 85.552) (width 1) (layer "F.Cu") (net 6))
 (segment (start 75.698 69.289874) (end 75.698001 80.910628) (width 1) (layer "F.Cu") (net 6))
 (segment (start 102.046501 67.207001) (end 77.780872 67.207001) (width 1) (layer "F.Cu") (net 6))
 (segment (start 84.78306 85.552) (end 87.434061 88.203) (width 1) (layer "F.Cu") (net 6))
 (segment (start 105.835 72.21) (end 105.835 70.9955) (width 1) (layer "F.Cu") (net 6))
 (segment (start 139.25 88) (end 139.15 87.9) (width 0.4) (layer "F.Cu") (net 14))
 (segment (start 107.187286 98.4695) (end 109.3 96.356786) (width 0.4) (layer "F.Cu") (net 14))
 (segment (start 95.5845 95.4875) (end 95.5845 96.5575) (width 0.4) (layer "F.Cu") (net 14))
 (segment (start 97.4965 98.4695) (end 107.187286 98.4695) (width 0.4) (layer "F.Cu") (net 14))
 (segment (start 139.15 87.9) (end 134.82 87.9) (width 0.4) (layer "F.Cu") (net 14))
 (segment (start 109.3 96.356786) (end 109.3 91) (width 0.4) (layer "F.Cu") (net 14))
 (segment (start 95.5845 96.5575) (end 97.4965 98.4695) (width 0.4) (layer "F.Cu") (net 14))
 (via (at 139.25 88) (size 1.4) (drill 0.85) (layers "F.Cu" "B.Cu") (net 14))
 (via (at 109.3 91) (size 1.4) (drill 0.85) (layers "F.Cu" "B.Cu") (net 14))
 (segment (start 136.25 91) (end 139.25 88) (width 0.4) (layer "B.Cu") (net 14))
 (segment (start 109.3 91) (end 136.25 91) (width 0.4) (layer "B.Cu") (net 14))
 (segment (start 95.7575 99.2705) (end 107.519072 99.2705) (width 0.4) (layer "F.Cu") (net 13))
 (segment (start 93.0445 95.4875) (end 93.0445 96.5575) (width 0.4) (layer "F.Cu") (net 13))
 (segment (start 107.519072 99.2705) (end 110.75 96.039572) (width 0.4) (layer "F.Cu") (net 13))
 (segment (start 93.0445 96.5575) (end 95.7575 99.2705) (width 0.4) (layer "F.Cu") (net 13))
 (segment (start 110.75 89.5) (end 112.35 87.9) (width 0.4) (layer "F.Cu") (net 13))
 (segment (start 110.75 96.039572) (end 110.75 89.5) (width 0.4) (layer "F.Cu") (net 13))
 (segment (start 112.35 87.9) (end 119.585 87.9) (width 0.4) (layer "F.Cu") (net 13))
 (segment (start 89.175 84) (end 115.663 84) (width 1) (layer "F.Cu") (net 22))
 (segment (start 115.663 84) (end 117.023 85.36) (width 1) (layer "F.Cu") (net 22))
 (segment (start 84.085 78.91) (end 89.175 84) (width 1) (layer "F.Cu") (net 22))
 (segment (start 117.023 85.36) (end 119.585 85.36) (width 1) (layer "F.Cu") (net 22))
 (segment (start 98.044 81.119) (end 118.746 81.119) (width 1) (layer "F.Cu") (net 9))
 (segment (start 118.746 81.119) (end 119.585 80.28) (width 1) (layer "F.Cu") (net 9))
 (segment (start 95.585 78.66) (end 98.044 81.119) (width 1) (layer "F.Cu") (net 9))
 (segment (start 106.585 78.66) (end 107.505 77.74) (width 1) (layer "F.Cu") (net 1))
 (segment (start 107.505 77.74) (end 119.585 77.74) (width 1) (layer "F.Cu") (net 1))
 (segment (start 103.295 72.21) (end 103.295 75.62) (width 1) (layer "F.Cu") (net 2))
 (segment (start 103.295 75.62) (end 103.585 75.91) (width 1) (layer "F.Cu") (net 2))
 (segment (start 103.585 75.91) (end 103.585 78.66) (width 1) (layer "F.Cu") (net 2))
 (segment (start 92.585 75.66) (end 92.585 78.66) (width 1) (layer "F.Cu") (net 7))
 (segment (start 92.335 75.41) (end 92.585 75.66) (width 1) (layer "F.Cu") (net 7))
 (segment (start 92.335 72.16) (end 92.335 75.41) (width 1) (layer "F.Cu") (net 7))
 (segment (start 80.795 75.71) (end 81.045 75.96) (width 1) (layer "F.Cu") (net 3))
 (segment (start 81.045 75.96) (end 81.045 78.87) (width 1) (layer "F.Cu") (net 3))
 (segment (start 80.795 71.91) (end 80.795 75.71) (width 1) (layer "F.Cu") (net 3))
 (segment (start 81.045 78.87) (end 81.085 78.91) (width 1) (layer "F.Cu") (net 3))
 (segment (start 113.252 94.498) (end 113.849 93.901) (width 1) (layer "F.Cu") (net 11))
 (segment (start 91.198186 101.7725) (end 108.555434 101.7725) (width 1) (layer "F.Cu") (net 11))
 (segment (start 153.651 92.330314) (end 153.651 92.173156) (width 1) (layer "F.Cu") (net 11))
 (segment (start 108.555434 101.7725) (end 113.252 97.075935) (width 1) (layer "F.Cu") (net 11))
 (segment (start 90.335 101.75) (end 91.175687 101.75) (width 1) (layer "F.Cu") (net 11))
 (segment (start 159.237 70.074398) (end 157.390601 68.228) (width 1) (layer "F.Cu") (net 11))
 (segment (start 153.824156 92) (end 158 92) (width 1) (layer "F.Cu") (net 11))
 (segment (start 85.4245 95.4875) (end 85.4245 96.8395) (width 1) (layer "F.Cu") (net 11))
 (segment (start 157.390601 68.228) (end 139.252 68.228) (width 1) (layer "F.Cu") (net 11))
 (segment (start 159.237 90.763) (end 159.237 70.074398) (width 1) (layer "F.Cu") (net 11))
 (segment (start 139.252 68.228) (end 134.82 72.66) (width 1) (layer "F.Cu") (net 11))
 (segment (start 113.849 93.901) (end 152.080314 93.901) (width 1) (layer "F.Cu") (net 11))
 (segment (start 152.080314 93.901) (end 153.651 92.330314) (width 1) (layer "F.Cu") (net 11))
 (segment (start 158 92) (end 159.237 90.763) (width 1) (layer "F.Cu") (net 11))
 (segment (start 113.252 97.075935) (end 113.252 94.498) (width 1) (layer "F.Cu") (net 11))
 (segment (start 91.175687 101.75) (end 91.198186 101.7725) (width 1) (layer "F.Cu") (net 11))
 (segment (start 153.651 92.173156) (end 153.824156 92) (width 1) (layer "F.Cu") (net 11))
 (segment (start 85.4245 96.8395) (end 90.335 101.75) (width 1) (layer "F.Cu") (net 11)))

